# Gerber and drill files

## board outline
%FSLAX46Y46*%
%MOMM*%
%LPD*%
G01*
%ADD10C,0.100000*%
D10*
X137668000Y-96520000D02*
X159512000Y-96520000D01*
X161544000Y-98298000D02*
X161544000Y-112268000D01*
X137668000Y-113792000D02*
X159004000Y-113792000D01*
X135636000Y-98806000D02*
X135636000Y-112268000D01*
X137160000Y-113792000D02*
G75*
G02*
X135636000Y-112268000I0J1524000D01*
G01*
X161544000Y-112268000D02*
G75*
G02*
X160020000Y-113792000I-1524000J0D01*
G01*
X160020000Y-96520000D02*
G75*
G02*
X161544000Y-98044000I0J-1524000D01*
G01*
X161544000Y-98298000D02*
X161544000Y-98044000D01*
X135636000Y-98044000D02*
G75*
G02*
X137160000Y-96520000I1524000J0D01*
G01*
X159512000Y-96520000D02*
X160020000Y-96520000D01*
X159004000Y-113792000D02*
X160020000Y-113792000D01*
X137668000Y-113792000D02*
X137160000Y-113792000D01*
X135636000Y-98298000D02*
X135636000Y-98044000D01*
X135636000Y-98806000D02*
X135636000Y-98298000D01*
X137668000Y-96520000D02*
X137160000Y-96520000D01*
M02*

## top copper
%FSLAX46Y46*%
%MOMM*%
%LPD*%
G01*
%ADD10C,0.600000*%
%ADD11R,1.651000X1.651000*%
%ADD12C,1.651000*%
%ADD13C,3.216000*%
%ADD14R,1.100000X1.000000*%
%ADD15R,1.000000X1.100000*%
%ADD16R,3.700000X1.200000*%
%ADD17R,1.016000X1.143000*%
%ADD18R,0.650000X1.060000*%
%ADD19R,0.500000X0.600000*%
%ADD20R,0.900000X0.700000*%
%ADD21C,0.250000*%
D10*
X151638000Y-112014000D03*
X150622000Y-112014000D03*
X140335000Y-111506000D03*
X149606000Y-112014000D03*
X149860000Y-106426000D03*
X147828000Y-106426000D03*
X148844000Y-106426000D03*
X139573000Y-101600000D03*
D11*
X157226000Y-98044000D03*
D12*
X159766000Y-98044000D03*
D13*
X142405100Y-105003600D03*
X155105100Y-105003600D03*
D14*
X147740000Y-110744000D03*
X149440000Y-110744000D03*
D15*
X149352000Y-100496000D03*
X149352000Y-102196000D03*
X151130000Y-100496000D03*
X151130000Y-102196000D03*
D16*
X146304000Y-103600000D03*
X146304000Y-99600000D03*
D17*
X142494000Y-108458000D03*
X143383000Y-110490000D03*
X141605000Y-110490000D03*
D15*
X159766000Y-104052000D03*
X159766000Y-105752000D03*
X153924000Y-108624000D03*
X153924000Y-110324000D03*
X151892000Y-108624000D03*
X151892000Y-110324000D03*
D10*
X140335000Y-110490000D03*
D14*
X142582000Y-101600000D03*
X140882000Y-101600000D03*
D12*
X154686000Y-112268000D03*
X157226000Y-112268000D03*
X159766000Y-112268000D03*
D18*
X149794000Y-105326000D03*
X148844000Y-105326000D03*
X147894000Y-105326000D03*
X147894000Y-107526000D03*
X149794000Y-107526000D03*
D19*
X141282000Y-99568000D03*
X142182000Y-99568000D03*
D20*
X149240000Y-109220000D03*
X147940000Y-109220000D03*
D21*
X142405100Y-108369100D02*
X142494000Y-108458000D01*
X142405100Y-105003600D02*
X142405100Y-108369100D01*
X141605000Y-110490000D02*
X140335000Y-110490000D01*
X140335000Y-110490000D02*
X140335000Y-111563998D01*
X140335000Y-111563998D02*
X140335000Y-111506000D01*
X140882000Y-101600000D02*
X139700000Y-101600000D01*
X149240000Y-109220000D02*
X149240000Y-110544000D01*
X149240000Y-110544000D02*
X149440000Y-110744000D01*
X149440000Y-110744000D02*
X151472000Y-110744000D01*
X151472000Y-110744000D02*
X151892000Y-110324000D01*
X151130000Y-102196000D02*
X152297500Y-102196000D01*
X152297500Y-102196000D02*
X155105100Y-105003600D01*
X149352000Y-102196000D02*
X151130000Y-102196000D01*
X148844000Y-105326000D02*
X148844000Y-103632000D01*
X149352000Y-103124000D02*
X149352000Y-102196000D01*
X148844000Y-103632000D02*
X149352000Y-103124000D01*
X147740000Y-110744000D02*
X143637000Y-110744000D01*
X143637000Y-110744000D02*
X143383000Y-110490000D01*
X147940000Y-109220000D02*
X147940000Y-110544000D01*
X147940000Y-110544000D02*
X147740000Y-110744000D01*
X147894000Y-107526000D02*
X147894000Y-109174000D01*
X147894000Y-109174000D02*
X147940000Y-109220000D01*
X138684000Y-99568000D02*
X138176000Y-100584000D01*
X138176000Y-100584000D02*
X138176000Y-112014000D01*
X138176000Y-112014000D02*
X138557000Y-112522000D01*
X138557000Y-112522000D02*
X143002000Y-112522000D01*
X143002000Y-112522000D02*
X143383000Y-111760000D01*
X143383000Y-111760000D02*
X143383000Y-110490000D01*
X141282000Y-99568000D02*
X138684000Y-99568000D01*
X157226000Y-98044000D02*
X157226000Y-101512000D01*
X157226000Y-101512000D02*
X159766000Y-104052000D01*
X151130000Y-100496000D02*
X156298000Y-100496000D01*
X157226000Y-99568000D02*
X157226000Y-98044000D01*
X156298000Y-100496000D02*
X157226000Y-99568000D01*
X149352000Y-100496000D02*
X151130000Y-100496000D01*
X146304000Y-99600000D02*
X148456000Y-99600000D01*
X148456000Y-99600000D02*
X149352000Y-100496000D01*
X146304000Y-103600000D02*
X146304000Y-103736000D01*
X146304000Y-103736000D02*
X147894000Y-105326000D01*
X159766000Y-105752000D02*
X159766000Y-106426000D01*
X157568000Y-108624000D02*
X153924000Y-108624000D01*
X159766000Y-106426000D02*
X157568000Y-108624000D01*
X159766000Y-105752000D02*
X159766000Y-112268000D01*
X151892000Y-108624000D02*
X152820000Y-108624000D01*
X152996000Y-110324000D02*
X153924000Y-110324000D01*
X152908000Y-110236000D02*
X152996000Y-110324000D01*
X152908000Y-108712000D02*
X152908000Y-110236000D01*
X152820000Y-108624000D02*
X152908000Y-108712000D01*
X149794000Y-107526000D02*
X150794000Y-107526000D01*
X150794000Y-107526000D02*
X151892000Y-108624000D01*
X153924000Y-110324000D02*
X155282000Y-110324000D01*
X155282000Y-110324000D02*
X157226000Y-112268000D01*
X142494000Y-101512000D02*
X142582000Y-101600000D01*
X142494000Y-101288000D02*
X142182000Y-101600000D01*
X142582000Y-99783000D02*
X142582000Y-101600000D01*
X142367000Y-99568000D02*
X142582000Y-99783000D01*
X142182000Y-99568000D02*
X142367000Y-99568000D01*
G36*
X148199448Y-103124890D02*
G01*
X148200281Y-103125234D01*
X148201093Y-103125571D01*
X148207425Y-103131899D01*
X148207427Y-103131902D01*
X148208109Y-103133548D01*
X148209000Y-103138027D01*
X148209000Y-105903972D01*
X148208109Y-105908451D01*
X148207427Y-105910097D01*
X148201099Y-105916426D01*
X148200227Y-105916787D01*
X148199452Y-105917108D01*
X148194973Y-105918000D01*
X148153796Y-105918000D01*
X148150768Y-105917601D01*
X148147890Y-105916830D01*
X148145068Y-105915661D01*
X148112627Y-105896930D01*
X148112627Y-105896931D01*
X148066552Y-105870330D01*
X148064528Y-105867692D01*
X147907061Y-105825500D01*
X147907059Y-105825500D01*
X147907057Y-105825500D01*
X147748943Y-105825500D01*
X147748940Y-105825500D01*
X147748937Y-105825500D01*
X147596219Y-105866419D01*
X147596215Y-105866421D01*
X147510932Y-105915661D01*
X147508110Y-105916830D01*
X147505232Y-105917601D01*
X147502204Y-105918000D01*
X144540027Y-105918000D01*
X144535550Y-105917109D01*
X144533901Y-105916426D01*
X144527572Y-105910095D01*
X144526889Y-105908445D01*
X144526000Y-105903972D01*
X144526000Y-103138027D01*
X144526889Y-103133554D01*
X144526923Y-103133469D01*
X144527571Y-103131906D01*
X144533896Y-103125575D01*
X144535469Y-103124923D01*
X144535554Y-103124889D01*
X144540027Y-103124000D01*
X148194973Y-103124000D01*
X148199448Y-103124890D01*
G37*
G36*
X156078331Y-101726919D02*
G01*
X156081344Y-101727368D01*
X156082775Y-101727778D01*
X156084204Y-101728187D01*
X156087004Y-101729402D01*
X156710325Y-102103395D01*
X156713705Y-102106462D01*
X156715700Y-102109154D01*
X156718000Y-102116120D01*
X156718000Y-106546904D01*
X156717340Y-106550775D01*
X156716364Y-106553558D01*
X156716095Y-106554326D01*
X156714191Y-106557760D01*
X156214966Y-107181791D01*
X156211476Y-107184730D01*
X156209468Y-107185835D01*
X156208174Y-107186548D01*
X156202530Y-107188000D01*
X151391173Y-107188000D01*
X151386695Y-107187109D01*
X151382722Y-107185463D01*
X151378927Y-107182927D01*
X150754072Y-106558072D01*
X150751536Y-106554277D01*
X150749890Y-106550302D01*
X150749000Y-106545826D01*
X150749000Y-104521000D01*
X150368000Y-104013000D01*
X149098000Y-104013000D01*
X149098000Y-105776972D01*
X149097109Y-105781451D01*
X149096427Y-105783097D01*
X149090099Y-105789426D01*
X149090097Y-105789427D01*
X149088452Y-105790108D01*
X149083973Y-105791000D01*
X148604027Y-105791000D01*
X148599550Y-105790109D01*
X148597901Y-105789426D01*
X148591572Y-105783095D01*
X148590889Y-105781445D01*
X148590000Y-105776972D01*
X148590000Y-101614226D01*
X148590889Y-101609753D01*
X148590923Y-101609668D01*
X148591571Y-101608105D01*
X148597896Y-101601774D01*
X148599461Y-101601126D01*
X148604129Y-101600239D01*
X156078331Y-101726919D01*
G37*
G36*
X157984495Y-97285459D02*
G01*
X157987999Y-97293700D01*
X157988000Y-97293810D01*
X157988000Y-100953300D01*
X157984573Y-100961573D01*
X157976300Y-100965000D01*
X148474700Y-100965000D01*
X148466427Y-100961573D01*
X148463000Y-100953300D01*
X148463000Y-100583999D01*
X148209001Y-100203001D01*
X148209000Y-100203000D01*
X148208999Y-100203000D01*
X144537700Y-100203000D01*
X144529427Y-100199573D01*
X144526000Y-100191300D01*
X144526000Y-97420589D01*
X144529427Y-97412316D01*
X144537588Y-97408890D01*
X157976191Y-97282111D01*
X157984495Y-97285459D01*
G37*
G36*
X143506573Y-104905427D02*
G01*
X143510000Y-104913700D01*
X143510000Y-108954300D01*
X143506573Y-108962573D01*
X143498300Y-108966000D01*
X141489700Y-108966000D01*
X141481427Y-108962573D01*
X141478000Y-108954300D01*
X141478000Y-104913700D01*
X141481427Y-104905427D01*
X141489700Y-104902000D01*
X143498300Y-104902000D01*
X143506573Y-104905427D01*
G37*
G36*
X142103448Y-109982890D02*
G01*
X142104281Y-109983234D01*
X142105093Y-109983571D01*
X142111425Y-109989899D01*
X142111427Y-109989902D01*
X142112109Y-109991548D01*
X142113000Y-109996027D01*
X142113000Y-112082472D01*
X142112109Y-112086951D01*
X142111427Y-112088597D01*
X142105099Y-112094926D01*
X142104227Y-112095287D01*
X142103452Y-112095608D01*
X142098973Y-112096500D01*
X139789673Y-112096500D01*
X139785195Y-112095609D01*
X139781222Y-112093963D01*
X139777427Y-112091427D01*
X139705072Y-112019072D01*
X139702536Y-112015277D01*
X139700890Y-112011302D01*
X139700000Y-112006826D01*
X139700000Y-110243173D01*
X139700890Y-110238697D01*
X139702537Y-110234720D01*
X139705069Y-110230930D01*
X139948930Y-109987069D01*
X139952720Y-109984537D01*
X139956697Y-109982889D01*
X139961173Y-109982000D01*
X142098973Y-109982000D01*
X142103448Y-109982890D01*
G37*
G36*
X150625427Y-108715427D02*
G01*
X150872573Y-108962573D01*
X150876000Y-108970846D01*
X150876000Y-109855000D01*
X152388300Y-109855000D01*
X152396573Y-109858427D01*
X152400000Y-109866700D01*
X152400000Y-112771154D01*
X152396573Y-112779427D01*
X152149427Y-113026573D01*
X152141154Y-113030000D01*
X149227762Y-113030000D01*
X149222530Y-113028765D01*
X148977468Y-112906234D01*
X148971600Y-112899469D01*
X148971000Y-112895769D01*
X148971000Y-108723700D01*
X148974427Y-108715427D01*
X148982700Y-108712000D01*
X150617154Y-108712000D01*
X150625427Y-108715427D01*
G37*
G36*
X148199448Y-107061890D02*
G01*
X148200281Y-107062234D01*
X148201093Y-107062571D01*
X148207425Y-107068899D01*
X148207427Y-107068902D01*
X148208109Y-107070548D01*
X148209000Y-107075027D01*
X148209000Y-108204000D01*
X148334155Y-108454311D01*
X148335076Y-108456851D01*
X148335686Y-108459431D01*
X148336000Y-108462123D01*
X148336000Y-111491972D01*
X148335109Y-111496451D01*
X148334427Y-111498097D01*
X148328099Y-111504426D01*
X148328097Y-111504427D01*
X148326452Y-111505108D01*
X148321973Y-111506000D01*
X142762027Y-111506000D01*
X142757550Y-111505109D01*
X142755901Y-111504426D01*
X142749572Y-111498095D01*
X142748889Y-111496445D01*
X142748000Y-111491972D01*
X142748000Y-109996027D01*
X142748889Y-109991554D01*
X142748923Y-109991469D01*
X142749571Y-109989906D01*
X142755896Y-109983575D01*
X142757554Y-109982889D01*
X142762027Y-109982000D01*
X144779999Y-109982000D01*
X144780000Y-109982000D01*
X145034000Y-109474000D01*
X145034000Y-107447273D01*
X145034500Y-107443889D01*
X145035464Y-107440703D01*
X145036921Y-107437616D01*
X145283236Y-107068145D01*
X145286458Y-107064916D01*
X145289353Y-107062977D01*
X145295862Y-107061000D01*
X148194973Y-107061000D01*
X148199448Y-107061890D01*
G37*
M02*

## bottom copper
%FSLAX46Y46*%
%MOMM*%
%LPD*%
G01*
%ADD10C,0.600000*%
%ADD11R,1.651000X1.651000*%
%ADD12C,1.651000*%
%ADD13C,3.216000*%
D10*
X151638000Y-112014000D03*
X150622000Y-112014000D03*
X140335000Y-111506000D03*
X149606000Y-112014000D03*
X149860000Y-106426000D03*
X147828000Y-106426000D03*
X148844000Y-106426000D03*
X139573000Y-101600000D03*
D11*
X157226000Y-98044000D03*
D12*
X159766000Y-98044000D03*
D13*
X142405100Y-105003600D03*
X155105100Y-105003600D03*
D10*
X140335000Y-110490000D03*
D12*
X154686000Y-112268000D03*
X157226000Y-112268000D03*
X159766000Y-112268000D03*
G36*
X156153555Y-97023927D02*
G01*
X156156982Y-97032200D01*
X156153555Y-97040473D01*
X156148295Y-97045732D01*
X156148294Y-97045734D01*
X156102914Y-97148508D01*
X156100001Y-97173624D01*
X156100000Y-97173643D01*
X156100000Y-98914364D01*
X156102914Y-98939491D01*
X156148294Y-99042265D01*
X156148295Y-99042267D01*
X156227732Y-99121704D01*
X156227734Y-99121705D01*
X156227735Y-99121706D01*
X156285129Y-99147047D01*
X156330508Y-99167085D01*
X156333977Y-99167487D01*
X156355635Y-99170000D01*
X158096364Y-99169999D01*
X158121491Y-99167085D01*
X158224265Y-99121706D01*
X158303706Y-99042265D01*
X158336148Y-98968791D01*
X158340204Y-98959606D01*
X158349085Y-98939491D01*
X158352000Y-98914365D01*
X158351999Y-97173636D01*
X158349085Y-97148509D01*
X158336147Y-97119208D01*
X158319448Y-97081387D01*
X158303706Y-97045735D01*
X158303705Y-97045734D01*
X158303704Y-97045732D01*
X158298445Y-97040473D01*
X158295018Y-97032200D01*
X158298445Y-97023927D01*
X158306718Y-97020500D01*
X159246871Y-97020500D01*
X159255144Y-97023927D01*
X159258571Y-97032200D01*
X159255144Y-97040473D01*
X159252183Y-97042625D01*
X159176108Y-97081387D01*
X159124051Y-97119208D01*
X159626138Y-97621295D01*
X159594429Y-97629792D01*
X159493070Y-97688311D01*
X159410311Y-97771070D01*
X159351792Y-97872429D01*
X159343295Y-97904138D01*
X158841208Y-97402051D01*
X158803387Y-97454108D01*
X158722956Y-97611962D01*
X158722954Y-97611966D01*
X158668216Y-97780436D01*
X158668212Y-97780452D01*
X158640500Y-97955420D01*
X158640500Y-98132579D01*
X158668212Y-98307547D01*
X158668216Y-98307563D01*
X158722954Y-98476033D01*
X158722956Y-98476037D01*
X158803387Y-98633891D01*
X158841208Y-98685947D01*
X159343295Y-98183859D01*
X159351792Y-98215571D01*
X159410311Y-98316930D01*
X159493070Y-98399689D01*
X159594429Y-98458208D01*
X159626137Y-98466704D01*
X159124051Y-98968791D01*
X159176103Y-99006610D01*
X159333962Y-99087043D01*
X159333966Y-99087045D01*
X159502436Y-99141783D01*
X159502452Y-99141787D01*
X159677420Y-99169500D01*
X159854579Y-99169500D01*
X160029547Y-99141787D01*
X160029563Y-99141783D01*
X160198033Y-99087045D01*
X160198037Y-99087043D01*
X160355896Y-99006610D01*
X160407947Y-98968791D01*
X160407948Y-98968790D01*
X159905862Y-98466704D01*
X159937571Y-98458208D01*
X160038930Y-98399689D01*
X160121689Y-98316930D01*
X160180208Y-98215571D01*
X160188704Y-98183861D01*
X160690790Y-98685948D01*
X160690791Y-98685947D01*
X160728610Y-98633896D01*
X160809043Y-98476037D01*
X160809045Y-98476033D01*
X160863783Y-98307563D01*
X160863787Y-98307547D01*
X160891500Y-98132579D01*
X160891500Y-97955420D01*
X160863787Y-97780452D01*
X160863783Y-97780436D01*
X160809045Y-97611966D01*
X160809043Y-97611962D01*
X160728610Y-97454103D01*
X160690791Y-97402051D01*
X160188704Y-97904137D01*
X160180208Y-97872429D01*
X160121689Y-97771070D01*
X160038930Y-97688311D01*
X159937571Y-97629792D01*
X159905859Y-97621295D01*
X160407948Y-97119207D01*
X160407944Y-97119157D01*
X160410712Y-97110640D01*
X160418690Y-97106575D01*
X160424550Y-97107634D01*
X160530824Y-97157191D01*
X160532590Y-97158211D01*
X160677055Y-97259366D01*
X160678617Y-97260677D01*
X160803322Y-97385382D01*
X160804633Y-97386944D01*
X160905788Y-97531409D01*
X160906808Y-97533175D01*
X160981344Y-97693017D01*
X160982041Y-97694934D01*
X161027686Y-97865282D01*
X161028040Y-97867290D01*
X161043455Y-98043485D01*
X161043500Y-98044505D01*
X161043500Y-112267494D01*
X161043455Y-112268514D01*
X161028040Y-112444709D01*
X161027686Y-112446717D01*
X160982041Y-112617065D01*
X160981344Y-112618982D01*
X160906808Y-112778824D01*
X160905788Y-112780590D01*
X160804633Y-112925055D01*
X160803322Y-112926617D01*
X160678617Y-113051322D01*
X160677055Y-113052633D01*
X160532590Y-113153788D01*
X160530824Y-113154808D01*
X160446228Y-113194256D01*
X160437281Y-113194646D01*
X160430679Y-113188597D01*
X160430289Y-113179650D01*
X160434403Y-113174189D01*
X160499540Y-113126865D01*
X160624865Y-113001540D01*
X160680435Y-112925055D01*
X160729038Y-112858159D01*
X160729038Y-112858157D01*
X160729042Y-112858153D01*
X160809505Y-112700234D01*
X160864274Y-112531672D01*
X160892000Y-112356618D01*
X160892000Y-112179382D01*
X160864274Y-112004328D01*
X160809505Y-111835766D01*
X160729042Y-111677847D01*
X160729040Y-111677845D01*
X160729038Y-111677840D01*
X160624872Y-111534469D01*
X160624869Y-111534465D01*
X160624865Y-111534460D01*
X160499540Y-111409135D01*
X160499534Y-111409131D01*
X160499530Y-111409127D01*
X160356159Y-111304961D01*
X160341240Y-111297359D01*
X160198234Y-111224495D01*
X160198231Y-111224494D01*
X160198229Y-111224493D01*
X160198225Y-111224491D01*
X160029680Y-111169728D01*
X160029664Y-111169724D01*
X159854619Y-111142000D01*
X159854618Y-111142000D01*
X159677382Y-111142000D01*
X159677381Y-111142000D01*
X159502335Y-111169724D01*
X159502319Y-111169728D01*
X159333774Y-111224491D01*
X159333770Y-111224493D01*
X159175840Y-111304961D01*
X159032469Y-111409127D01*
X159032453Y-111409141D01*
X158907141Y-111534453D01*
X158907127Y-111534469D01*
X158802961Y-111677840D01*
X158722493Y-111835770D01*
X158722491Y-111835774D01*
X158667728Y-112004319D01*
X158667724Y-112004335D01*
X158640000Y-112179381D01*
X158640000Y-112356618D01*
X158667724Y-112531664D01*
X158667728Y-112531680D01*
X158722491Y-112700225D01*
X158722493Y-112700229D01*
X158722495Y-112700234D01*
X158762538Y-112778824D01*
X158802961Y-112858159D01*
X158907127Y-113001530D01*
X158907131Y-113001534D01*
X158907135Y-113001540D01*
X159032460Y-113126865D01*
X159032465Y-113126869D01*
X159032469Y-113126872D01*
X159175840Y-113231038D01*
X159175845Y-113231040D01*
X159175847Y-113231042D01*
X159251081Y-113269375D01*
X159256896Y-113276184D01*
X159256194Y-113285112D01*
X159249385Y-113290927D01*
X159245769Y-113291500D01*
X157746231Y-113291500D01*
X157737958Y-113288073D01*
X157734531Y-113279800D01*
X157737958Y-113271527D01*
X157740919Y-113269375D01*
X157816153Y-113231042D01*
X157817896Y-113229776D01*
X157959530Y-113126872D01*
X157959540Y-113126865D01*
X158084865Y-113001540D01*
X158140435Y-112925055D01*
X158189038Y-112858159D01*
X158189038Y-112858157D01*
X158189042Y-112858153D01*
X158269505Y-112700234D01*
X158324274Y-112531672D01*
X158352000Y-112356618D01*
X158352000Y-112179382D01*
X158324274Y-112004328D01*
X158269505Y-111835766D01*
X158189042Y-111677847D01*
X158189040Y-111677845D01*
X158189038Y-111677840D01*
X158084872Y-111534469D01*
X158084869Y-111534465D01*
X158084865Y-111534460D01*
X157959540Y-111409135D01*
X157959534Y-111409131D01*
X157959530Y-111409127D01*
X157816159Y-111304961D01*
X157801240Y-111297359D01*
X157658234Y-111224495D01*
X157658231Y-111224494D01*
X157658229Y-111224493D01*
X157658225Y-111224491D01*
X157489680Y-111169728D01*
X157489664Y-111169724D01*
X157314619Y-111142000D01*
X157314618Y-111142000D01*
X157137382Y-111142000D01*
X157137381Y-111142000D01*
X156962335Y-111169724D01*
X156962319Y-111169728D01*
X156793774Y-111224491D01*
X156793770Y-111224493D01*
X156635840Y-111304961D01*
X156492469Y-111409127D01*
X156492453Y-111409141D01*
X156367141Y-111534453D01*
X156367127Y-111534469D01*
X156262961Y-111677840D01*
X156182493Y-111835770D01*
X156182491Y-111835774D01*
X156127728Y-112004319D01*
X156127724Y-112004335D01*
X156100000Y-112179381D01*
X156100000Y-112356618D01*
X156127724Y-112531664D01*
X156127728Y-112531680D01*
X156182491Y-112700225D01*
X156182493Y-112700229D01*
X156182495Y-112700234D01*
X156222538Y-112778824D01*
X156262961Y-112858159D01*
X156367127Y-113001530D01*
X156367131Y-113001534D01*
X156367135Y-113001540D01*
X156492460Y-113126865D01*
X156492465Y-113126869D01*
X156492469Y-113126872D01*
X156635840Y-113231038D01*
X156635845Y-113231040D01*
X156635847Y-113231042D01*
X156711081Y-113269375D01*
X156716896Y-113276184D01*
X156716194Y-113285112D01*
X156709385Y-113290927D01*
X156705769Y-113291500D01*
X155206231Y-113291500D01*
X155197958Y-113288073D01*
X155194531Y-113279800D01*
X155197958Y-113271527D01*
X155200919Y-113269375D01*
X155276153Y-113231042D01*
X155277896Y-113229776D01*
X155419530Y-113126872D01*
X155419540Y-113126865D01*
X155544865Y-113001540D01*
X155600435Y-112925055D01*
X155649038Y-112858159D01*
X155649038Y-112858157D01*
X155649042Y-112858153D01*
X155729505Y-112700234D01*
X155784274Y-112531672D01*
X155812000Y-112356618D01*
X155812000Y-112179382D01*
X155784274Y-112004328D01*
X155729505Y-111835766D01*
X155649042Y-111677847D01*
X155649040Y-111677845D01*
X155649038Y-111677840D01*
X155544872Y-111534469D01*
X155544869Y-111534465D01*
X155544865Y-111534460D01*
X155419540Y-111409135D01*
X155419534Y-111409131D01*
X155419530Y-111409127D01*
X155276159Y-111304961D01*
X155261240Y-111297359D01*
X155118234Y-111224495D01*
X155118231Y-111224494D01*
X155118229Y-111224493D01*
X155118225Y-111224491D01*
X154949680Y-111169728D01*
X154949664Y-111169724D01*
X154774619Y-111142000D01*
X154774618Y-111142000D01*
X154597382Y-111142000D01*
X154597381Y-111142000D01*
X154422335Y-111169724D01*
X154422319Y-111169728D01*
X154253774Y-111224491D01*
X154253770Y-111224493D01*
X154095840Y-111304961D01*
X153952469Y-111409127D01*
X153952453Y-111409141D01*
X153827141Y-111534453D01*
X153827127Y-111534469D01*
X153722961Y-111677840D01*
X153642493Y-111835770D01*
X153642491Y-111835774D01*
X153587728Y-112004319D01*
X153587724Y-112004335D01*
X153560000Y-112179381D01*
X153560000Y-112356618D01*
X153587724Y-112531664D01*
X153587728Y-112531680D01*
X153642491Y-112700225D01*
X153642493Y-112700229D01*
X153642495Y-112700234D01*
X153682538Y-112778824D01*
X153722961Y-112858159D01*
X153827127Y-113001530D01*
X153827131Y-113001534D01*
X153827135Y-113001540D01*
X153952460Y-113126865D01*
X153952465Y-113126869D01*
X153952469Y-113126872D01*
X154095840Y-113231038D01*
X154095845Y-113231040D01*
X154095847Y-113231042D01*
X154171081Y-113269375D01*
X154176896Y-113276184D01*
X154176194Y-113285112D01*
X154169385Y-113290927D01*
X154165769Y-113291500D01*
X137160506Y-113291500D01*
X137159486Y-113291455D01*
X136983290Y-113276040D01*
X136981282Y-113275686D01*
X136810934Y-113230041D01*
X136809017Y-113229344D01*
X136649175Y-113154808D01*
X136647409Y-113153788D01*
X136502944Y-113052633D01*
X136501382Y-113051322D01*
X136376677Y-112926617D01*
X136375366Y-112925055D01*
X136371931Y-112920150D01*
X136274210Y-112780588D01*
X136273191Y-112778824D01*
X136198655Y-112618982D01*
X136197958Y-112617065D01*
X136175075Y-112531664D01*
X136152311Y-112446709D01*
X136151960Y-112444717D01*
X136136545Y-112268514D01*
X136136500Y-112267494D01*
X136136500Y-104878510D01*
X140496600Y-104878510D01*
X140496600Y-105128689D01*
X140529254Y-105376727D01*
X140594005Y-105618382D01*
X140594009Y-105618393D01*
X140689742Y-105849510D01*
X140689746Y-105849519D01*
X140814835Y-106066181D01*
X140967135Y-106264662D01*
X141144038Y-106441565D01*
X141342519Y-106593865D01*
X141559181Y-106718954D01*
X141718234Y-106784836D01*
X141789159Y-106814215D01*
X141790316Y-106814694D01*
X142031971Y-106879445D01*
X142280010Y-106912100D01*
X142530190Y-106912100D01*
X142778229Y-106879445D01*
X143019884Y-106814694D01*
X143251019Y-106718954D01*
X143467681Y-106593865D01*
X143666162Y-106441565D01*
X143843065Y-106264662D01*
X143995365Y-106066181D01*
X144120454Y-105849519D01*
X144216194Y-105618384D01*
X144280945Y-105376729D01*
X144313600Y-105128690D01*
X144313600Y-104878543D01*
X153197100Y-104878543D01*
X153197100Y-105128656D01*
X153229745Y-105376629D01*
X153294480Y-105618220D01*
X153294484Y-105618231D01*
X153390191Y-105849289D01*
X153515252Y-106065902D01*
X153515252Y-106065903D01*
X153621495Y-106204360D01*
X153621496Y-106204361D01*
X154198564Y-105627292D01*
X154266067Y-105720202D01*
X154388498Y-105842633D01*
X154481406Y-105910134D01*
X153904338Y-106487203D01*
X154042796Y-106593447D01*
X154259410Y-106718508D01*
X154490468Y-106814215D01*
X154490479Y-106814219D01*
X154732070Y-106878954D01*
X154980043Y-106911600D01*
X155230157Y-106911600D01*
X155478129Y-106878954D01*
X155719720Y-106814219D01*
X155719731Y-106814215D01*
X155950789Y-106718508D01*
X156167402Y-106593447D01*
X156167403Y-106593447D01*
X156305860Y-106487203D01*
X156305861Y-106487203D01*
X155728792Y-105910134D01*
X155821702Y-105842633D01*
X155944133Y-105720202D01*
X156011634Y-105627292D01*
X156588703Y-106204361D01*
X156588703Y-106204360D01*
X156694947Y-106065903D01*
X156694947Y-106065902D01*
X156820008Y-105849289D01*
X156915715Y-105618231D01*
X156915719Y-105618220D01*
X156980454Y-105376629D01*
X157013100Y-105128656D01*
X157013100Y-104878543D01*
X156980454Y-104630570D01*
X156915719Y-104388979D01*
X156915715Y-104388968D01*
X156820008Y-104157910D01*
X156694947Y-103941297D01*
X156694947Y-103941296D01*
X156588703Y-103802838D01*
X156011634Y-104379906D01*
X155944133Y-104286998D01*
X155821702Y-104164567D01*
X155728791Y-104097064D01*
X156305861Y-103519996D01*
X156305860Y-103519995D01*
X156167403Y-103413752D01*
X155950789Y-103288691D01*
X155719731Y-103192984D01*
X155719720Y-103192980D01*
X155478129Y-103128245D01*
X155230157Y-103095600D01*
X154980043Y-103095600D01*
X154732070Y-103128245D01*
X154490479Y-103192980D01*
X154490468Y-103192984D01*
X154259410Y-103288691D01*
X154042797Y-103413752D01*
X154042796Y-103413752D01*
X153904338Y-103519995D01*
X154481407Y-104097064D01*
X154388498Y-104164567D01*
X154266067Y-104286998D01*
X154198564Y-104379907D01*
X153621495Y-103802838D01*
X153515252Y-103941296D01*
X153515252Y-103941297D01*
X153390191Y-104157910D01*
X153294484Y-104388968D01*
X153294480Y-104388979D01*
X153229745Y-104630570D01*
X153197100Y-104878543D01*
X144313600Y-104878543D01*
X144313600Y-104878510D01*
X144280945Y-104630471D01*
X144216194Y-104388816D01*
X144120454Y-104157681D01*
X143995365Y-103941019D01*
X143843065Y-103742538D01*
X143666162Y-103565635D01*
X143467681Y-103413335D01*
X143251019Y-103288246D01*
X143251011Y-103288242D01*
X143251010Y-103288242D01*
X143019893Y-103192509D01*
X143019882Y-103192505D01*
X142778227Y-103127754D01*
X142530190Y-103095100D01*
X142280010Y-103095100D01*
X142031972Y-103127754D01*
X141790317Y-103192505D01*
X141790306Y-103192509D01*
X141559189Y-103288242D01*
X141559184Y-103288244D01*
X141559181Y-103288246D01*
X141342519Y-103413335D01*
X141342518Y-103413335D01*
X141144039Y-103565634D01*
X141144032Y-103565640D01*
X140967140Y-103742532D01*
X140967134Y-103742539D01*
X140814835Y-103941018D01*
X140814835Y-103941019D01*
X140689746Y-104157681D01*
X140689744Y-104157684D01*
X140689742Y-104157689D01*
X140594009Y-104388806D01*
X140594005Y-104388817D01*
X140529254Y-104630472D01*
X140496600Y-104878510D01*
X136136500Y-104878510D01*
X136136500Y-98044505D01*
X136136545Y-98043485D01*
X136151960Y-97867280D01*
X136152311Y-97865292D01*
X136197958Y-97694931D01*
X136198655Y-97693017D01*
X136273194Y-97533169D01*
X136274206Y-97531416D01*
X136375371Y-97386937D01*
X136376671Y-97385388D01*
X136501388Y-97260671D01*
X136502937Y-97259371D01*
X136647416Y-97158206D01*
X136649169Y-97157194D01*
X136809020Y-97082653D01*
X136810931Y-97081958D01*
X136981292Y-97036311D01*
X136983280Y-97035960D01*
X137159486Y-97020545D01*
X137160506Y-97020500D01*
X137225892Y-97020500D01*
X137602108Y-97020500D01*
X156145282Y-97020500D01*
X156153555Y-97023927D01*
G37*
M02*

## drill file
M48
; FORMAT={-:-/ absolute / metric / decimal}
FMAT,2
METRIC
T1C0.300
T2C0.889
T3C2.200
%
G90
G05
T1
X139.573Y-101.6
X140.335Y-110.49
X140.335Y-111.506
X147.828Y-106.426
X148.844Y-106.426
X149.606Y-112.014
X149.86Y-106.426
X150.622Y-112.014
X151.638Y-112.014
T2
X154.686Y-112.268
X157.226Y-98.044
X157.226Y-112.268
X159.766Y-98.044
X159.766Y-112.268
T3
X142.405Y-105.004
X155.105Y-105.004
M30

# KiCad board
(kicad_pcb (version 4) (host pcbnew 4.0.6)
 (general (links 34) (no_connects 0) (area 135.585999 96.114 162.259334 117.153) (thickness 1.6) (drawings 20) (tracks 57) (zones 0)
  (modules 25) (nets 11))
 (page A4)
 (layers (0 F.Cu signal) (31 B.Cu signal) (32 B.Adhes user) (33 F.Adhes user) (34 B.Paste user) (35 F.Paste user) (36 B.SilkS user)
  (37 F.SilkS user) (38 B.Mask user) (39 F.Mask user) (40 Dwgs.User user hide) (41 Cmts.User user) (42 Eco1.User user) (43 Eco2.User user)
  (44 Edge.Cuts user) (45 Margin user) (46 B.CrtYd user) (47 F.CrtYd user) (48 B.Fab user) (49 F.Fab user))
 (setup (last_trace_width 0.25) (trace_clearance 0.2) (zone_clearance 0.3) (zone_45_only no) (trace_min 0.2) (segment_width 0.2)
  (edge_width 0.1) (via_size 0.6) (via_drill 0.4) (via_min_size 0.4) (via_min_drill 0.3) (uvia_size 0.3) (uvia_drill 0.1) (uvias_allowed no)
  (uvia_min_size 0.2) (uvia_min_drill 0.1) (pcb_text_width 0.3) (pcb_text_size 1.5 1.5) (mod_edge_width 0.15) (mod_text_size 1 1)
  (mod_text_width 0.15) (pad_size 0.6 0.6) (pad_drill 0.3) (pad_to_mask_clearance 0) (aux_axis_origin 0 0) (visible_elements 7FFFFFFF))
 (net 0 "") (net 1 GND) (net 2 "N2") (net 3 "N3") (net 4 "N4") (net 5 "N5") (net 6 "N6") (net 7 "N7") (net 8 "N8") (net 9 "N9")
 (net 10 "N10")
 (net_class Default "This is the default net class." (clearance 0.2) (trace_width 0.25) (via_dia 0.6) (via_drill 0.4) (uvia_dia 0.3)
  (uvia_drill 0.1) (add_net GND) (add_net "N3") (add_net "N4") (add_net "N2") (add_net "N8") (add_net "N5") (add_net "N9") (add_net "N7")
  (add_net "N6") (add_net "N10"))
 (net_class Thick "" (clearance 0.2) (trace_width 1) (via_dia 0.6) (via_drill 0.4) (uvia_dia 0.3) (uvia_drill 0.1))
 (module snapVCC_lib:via (layer F.Cu) (at 151.638 112.014)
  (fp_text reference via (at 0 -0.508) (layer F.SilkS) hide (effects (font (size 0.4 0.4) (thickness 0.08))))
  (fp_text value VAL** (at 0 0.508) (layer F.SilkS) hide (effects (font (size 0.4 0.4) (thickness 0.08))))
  (pad 1 thru_hole circle (at 0 0) (size 0.6 0.6) (drill 0.3) (layers *.Cu) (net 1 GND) (zone_connect 2)))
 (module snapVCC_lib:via (layer F.Cu) (at 150.622 112.014)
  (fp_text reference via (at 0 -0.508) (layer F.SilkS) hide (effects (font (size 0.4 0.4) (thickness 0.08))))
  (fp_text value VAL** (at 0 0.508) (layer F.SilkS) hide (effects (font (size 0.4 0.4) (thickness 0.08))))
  (pad 1 thru_hole circle (at 0 0) (size 0.6 0.6) (drill 0.3) (layers *.Cu) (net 1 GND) (zone_connect 2)))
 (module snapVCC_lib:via (layer F.Cu) (at 140.335 111.506)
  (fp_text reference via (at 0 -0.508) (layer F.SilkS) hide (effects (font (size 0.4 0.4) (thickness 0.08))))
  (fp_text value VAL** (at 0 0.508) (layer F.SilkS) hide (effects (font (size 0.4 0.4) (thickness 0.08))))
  (pad 1 thru_hole circle (at 0 0) (size 0.6 0.6) (drill 0.3) (layers *.Cu) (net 1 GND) (zone_connect 2)))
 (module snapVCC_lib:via (layer F.Cu) (at 149.606 112.014)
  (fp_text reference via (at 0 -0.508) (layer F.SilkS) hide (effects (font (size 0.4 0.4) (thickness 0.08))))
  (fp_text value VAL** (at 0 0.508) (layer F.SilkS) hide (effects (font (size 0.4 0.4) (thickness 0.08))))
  (pad 1 thru_hole circle (at 0 0) (size 0.6 0.6) (drill 0.3) (layers *.Cu) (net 1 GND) (zone_connect 2)))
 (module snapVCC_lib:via (layer F.Cu) (at 149.86 106.426)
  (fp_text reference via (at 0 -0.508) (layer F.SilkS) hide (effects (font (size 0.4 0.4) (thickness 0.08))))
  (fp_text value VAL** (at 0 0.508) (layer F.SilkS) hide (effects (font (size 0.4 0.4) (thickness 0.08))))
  (pad 1 thru_hole circle (at 0 0) (size 0.6 0.6) (drill 0.3) (layers *.Cu) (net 1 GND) (zone_connect 2)))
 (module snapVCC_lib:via (layer F.Cu) (at 147.828 106.426)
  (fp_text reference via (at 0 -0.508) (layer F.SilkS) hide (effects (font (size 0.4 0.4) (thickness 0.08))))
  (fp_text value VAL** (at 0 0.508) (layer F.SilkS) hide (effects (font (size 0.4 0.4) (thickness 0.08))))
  (pad 1 thru_hole circle (at 0 0) (size 0.6 0.6) (drill 0.3) (layers *.Cu) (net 1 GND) (zone_connect 2)))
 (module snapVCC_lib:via (layer F.Cu) (at 148.844 106.426)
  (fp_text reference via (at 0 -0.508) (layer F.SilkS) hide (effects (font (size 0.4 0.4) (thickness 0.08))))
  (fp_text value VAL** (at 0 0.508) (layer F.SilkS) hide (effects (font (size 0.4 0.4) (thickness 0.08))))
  (pad 1 thru_hole circle (at 0 0) (size 0.6 0.6) (drill 0.3) (layers *.Cu) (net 1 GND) (zone_connect 2)))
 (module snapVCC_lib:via (layer F.Cu) (at 139.573 101.6)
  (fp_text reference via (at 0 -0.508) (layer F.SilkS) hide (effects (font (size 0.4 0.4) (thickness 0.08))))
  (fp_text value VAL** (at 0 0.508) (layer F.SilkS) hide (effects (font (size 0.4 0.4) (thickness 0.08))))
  (pad 1 thru_hole circle (at 0 0) (size 0.6 0.6) (drill 0.3) (layers *.Cu) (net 1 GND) (zone_connect 2)))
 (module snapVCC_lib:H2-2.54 (layer F.Cu) (at 158.496 98.044 90)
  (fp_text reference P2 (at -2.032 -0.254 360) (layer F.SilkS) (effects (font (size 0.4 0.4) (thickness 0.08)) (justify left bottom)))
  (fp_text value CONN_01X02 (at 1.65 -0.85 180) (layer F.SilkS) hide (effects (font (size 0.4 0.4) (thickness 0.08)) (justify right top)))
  (pad 1 thru_hole rect (at 0 -1.27 90) (size 1.651 1.651) (drill 0.889) (layers *.Cu *.Mask) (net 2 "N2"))
  (pad 2 thru_hole circle (at 0 1.27 90) (size 1.651 1.651) (drill 0.889) (layers *.Cu *.Mask) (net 1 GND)))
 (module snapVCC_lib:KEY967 (layer B.Cu) (at 148.7551 105.0036)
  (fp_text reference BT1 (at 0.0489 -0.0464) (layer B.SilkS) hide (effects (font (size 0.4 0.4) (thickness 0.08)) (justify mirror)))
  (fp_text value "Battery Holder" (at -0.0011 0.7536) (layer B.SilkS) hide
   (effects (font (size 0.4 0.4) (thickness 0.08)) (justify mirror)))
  (pad 1 thru_hole circle (at -6.35 0) (size 3.216 3.216) (drill 2.2) (layers *.Cu *.Mask) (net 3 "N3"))
  (pad 2 thru_hole circle (at 6.35 0) (size 3.216 3.216) (drill 2.2) (layers *.Cu *.Mask) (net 1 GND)))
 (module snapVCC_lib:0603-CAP (layer F.Cu) (at 148.59 110.744)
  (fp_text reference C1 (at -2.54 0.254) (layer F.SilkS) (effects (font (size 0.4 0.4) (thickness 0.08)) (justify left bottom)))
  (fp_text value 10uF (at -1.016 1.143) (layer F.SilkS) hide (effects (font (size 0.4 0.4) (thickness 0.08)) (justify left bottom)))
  (pad 1 smd rect (at -0.85 0) (size 1.1 1) (layers F.Cu F.Paste F.Mask) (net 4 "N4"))
  (pad 2 smd rect (at 0.85 0) (size 1.1 1) (layers F.Cu F.Paste F.Mask) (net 1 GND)))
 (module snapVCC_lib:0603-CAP (layer F.Cu) (at 149.352 101.346 270)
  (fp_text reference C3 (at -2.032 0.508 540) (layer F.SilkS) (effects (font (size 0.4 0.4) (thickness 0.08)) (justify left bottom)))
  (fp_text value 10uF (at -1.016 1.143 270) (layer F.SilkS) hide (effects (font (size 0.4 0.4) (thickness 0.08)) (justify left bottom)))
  (pad 1 smd rect (at -0.85 0 270) (size 1.1 1) (layers F.Cu F.Paste F.Mask) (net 2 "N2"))
  (pad 2 smd rect (at 0.85 0 270) (size 1.1 1) (layers F.Cu F.Paste F.Mask) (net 1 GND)))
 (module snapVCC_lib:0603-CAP (layer F.Cu) (at 151.13 101.346 270)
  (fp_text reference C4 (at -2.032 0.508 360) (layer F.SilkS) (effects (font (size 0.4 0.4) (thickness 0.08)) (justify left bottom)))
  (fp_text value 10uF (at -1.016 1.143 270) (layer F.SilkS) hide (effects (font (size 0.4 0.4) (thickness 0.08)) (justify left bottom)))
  (pad 1 smd rect (at -0.85 0 270) (size 1.1 1) (layers F.Cu F.Paste F.Mask) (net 2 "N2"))
  (pad 2 smd rect (at 0.85 0 270) (size 1.1 1) (layers F.Cu F.Paste F.Mask) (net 1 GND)))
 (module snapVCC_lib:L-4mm (layer F.Cu) (at 146.304 101.6 90)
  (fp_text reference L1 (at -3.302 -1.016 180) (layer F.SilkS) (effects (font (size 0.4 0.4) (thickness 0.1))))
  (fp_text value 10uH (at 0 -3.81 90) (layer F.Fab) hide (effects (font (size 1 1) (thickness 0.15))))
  (pad 1 smd rect (at -2 0 90) (size 1.2 3.7) (layers F.Cu F.Paste F.Mask) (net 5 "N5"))
  (pad 2 smd rect (at 2 0 90) (size 1.2 3.7) (layers F.Cu F.Paste F.Mask) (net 2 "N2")))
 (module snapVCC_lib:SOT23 (layer F.Cu) (at 142.494 109.474)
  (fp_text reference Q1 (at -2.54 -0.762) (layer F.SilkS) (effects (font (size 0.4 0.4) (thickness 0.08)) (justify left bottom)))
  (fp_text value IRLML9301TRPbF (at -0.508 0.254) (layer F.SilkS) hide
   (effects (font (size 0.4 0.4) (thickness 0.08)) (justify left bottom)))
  (pad 3 smd rect (at 0 -1.016) (size 1.016 1.143) (layers F.Cu F.Paste F.Mask) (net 3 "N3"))
  (pad 2 smd rect (at 0.889 1.016) (size 1.016 1.143) (layers F.Cu F.Paste F.Mask) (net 4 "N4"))
  (pad 1 smd rect (at -0.889 1.016 180) (size 1.016 1.143) (layers F.Cu F.Paste F.Mask) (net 1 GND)))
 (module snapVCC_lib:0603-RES (layer F.Cu) (at 159.766 104.902 270)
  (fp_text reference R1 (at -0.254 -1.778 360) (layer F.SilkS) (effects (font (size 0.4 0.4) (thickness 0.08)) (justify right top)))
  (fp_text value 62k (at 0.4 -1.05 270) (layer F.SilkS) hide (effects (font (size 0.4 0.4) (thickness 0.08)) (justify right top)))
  (pad 1 smd rect (at -0.85 0 270) (size 1.1 1) (layers F.Cu F.Paste F.Mask) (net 2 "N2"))
  (pad 2 smd rect (at 0.85 0 270) (size 1.1 1) (layers F.Cu F.Paste F.Mask) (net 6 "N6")))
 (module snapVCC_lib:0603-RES (layer F.Cu) (at 153.924 109.474 270)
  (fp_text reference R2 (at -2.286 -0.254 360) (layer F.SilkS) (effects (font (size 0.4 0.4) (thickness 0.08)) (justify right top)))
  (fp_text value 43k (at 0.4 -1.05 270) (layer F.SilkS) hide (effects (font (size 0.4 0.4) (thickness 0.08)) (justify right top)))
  (pad 1 smd rect (at -0.85 0 270) (size 1.1 1) (layers F.Cu F.Paste F.Mask) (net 6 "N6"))
  (pad 2 smd rect (at 0.85 0 270) (size 1.1 1) (layers F.Cu F.Paste F.Mask) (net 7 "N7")))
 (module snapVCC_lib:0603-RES (layer F.Cu) (at 151.892 109.474 270)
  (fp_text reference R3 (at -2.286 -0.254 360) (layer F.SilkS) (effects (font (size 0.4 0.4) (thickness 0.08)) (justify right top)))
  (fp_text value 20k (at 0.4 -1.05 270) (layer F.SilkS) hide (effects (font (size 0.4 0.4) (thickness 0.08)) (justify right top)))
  (pad 1 smd rect (at -0.85 0 270) (size 1.1 1) (layers F.Cu F.Paste F.Mask) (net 7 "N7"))
  (pad 2 smd rect (at 0.85 0 270) (size 1.1 1) (layers F.Cu F.Paste F.Mask) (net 1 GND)))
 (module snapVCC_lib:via (layer F.Cu) (at 140.335 110.49)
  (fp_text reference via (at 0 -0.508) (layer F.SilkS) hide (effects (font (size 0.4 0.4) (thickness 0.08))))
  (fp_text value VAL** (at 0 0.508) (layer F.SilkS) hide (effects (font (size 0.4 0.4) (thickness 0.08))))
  (pad 1 thru_hole circle (at 0 0) (size 0.6 0.6) (drill 0.3) (layers *.Cu) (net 1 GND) (zone_connect 2)))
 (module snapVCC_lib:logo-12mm (layer F.Cu) (at 138.049 105.156 90)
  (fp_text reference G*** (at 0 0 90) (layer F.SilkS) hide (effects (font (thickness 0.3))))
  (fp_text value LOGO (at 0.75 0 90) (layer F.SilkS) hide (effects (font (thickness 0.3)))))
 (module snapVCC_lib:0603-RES (layer F.Cu) (at 141.732 101.6 180)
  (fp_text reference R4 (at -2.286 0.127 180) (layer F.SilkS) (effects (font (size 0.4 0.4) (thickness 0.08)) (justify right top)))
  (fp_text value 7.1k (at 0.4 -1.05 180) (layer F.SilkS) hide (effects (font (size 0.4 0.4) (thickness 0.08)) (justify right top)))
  (pad 1 smd rect (at -0.85 0 180) (size 1.1 1) (layers F.Cu F.Paste F.Mask) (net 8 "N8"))
  (pad 2 smd rect (at 0.85 0 180) (size 1.1 1) (layers F.Cu F.Paste F.Mask) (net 1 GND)))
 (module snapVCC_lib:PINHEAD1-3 (layer F.Cu) (at 157.226 112.268)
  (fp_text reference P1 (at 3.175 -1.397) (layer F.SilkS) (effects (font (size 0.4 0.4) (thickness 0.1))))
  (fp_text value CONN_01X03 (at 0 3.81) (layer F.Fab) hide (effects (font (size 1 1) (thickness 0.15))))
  (pad 1 thru_hole circle (at -2.54 0) (size 1.651 1.651) (drill 0.889) (layers *.Cu *.Mask) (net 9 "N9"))
  (pad 2 thru_hole circle (at 0 0) (size 1.651 1.651) (drill 0.889) (layers *.Cu *.Mask) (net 7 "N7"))
  (pad 3 thru_hole circle (at 2.54 0) (size 1.651 1.651) (drill 0.889) (layers *.Cu *.Mask) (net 6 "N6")))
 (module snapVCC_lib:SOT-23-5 (layer F.Cu) (at 148.844 106.426 270)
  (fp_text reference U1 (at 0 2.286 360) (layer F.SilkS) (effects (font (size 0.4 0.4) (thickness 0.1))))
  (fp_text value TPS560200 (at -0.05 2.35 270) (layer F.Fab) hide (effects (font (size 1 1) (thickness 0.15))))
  (pad 1 smd rect (at -1.1 -0.95 270) (size 1.06 0.65) (layers F.Cu F.Paste F.Mask) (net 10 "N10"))
  (pad 2 smd rect (at -1.1 0 270) (size 1.06 0.65) (layers F.Cu F.Paste F.Mask) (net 1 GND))
  (pad 3 smd rect (at -1.1 0.95 270) (size 1.06 0.65) (layers F.Cu F.Paste F.Mask) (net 5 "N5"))
  (pad 4 smd rect (at 1.1 0.95 270) (size 1.06 0.65) (layers F.Cu F.Paste F.Mask) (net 4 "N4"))
  (pad 5 smd rect (at 1.1 -0.95 270) (size 1.06 0.65) (layers F.Cu F.Paste F.Mask) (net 7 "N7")))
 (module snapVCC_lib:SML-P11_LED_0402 (layer F.Cu) (at 141.732 99.568 180)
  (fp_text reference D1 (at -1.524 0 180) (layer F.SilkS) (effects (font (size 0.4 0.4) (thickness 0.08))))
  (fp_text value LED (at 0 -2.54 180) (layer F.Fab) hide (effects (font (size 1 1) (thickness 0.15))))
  (pad 2 smd rect (at 0.45 0 180) (size 0.5 0.6) (layers F.Cu F.Paste F.Mask) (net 4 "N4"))
  (pad 1 smd rect (at -0.45 0 180) (size 0.5 0.6) (layers F.Cu F.Paste F.Mask) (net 8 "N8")))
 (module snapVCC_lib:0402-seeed (layer F.Cu) (at 148.59 109.22)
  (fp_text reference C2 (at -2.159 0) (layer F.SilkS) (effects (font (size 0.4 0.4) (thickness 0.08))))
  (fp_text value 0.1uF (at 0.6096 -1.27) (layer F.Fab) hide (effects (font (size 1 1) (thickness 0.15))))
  (pad 2 smd rect (at 0.65 0) (size 0.9 0.7) (layers F.Cu F.Paste F.Mask) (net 1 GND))
  (pad 1 smd rect (at -0.65 0) (size 0.9 0.7) (layers F.Cu F.Paste F.Mask) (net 4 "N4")))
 (gr_line (start 137.668 96.52) (end 159.512 96.52) (angle 90) (layer Edge.Cuts) (width 0.1))
 (gr_line (start 161.544 98.298) (end 161.544 112.268) (angle 90) (layer Edge.Cuts) (width 0.1))
 (gr_line (start 137.668 113.792) (end 159.004 113.792) (angle 90) (layer Edge.Cuts) (width 0.1))
 (gr_line (start 135.636 98.806) (end 135.636 112.268) (angle 90) (layer Edge.Cuts) (width 0.1))
 (gr_arc (start 137.16 112.268) (end 137.16 113.792) (angle 90) (layer Edge.Cuts) (width 0.1))
 (gr_arc (start 160.02 112.268) (end 161.544 112.268) (angle 90) (layer Edge.Cuts) (width 0.1))
 (gr_arc (start 160.02 98.044) (end 160.02 96.52) (angle 90) (layer Edge.Cuts) (width 0.1))
 (gr_line (start 161.544 98.298) (end 161.544 98.044) (angle 90) (layer Edge.Cuts) (width 0.1))
 (gr_arc (start 137.16 98.044) (end 135.636 98.044) (angle 90) (layer Edge.Cuts) (width 0.1))
 (gr_line (start 159.512 96.52) (end 160.02 96.52) (angle 90) (layer Edge.Cuts) (width 0.1))
 (gr_line (start 159.004 113.792) (end 160.02 113.792) (angle 90) (layer Edge.Cuts) (width 0.1))
 (gr_line (start 137.668 113.792) (end 137.16 113.792) (angle 90) (layer Edge.Cuts) (width 0.1))
 (gr_line (start 135.636 98.298) (end 135.636 98.044) (angle 90) (layer Edge.Cuts) (width 0.1))
 (gr_line (start 135.636 98.806) (end 135.636 98.298) (angle 90) (layer Edge.Cuts) (width 0.1))
 (gr_line (start 137.668 96.52) (end 137.16 96.52) (angle 90) (layer Edge.Cuts) (width 0.1))
 (segment (start 142.4051 108.3691) (end 142.494 108.458) (width 0.25) (layer F.Cu) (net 3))
 (segment (start 142.4051 105.0036) (end 142.4051 108.3691) (width 0.25) (layer F.Cu) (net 3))
 (segment (start 141.605 110.49) (end 140.335 110.49) (width 0.25) (layer F.Cu) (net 1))
 (segment (start 140.335 110.49) (end 140.335 111.563998) (width 0.25) (layer F.Cu) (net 1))
 (segment (start 140.335 111.563998) (end 140.335 111.506) (width 0.25) (layer F.Cu) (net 1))
 (segment (start 140.882 101.6) (end 139.7 101.6) (width 0.25) (layer F.Cu) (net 1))
 (segment (start 149.24 109.22) (end 149.24 110.544) (width 0.25) (layer F.Cu) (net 1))
 (segment (start 149.24 110.544) (end 149.44 110.744) (width 0.25) (layer F.Cu) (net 1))
 (segment (start 149.44 110.744) (end 151.472 110.744) (width 0.25) (layer F.Cu) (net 1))
 (segment (start 151.472 110.744) (end 151.892 110.324) (width 0.25) (layer F.Cu) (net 1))
 (segment (start 151.13 102.196) (end 152.2975 102.196) (width 0.25) (layer F.Cu) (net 1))
 (segment (start 152.2975 102.196) (end 155.1051 105.0036) (width 0.25) (layer F.Cu) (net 1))
 (segment (start 149.352 102.196) (end 151.13 102.196) (width 0.25) (layer F.Cu) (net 1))
 (segment (start 148.844 105.326) (end 148.844 103.632) (width 0.25) (layer F.Cu) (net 1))
 (segment (start 149.352 103.124) (end 149.352 102.196) (width 0.25) (layer F.Cu) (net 1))
 (segment (start 148.844 103.632) (end 149.352 103.124) (width 0.25) (layer F.Cu) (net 1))
 (segment (start 147.74 110.744) (end 143.637 110.744) (width 0.25) (layer F.Cu) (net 4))
 (segment (start 143.637 110.744) (end 143.383 110.49) (width 0.25) (layer F.Cu) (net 4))
 (segment (start 147.94 109.22) (end 147.94 110.544) (width 0.25) (layer F.Cu) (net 4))
 (segment (start 147.94 110.544) (end 147.74 110.744) (width 0.25) (layer F.Cu) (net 4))
 (segment (start 147.894 107.526) (end 147.894 109.174) (width 0.25) (layer F.Cu) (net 4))
 (segment (start 147.894 109.174) (end 147.94 109.22) (width 0.25) (layer F.Cu) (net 4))
 (segment (start 138.684 99.568) (end 138.176 100.584) (width 0.25) (layer F.Cu) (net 4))
 (segment (start 138.176 100.584) (end 138.176 112.014) (width 0.25) (layer F.Cu) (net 4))
 (segment (start 138.176 112.014) (end 138.557 112.522) (width 0.25) (layer F.Cu) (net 4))
 (segment (start 138.557 112.522) (end 143.002 112.522) (width 0.25) (layer F.Cu) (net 4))
 (segment (start 143.002 112.522) (end 143.383 111.76) (width 0.25) (layer F.Cu) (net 4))
 (segment (start 143.383 111.76) (end 143.383 110.49) (width 0.25) (layer F.Cu) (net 4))
 (segment (start 141.282 99.568) (end 138.684 99.568) (width 0.25) (layer F.Cu) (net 4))
 (segment (start 157.226 98.044) (end 157.226 101.512) (width 0.25) (layer F.Cu) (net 2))
 (segment (start 157.226 101.512) (end 159.766 104.052) (width 0.25) (layer F.Cu) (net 2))
 (segment (start 151.13 100.496) (end 156.298 100.496) (width 0.25) (layer F.Cu) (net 2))
 (segment (start 157.226 99.568) (end 157.226 98.044) (width 0.25) (layer F.Cu) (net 2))
 (segment (start 156.298 100.496) (end 157.226 99.568) (width 0.25) (layer F.Cu) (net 2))
 (segment (start 149.352 100.496) (end 151.13 100.496) (width 0.25) (layer F.Cu) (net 2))
 (segment (start 146.304 99.6) (end 148.456 99.6) (width 0.25) (layer F.Cu) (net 2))
 (segment (start 148.456 99.6) (end 149.352 100.496) (width 0.25) (layer F.Cu) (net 2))
 (segment (start 146.304 103.6) (end 146.304 103.736) (width 0.25) (layer F.Cu) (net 5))
 (segment (start 146.304 103.736) (end 147.894 105.326) (width 0.25) (layer F.Cu) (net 5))
 (segment (start 159.766 105.752) (end 159.766 106.426) (width 0.25) (layer F.Cu) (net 6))
 (segment (start 157.568 108.624) (end 153.924 108.624) (width 0.25) (layer F.Cu) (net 6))
 (segment (start 159.766 106.426) (end 157.568 108.624) (width 0.25) (layer F.Cu) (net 6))
 (segment (start 159.766 105.752) (end 159.766 112.268) (width 0.25) (layer F.Cu) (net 6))
 (segment (start 151.892 108.624) (end 152.82 108.624) (width 0.25) (layer F.Cu) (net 7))
 (segment (start 152.996 110.324) (end 153.924 110.324) (width 0.25) (layer F.Cu) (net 7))
 (segment (start 152.908 110.236) (end 152.996 110.324) (width 0.25) (layer F.Cu) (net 7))
 (segment (start 152.908 108.712) (end 152.908 110.236) (width 0.25) (layer F.Cu) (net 7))
 (segment (start 152.82 108.624) (end 152.908 108.712) (width 0.25) (layer F.Cu) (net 7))
 (segment (start 149.794 107.526) (end 150.794 107.526) (width 0.25) (layer F.Cu) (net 7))
 (segment (start 150.794 107.526) (end 151.892 108.624) (width 0.25) (layer F.Cu) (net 7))
 (segment (start 153.924 110.324) (end 155.282 110.324) (width 0.25) (layer F.Cu) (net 7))
 (segment (start 155.282 110.324) (end 157.226 112.268) (width 0.25) (layer F.Cu) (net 7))
 (segment (start 142.494 101.512) (end 142.582 101.6) (width 0.25) (layer F.Cu) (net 8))
 (segment (start 142.494 101.288) (end 142.182 101.6) (width 0.25) (layer F.Cu) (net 8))
 (segment (start 142.582 99.783) (end 142.582 101.6) (width 0.25) (layer F.Cu) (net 8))
 (segment (start 142.367 99.568) (end 142.582 99.783) (width 0.25) (layer F.Cu) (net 8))
 (segment (start 142.182 99.568) (end 142.367 99.568) (width 0.25) (layer F.Cu) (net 8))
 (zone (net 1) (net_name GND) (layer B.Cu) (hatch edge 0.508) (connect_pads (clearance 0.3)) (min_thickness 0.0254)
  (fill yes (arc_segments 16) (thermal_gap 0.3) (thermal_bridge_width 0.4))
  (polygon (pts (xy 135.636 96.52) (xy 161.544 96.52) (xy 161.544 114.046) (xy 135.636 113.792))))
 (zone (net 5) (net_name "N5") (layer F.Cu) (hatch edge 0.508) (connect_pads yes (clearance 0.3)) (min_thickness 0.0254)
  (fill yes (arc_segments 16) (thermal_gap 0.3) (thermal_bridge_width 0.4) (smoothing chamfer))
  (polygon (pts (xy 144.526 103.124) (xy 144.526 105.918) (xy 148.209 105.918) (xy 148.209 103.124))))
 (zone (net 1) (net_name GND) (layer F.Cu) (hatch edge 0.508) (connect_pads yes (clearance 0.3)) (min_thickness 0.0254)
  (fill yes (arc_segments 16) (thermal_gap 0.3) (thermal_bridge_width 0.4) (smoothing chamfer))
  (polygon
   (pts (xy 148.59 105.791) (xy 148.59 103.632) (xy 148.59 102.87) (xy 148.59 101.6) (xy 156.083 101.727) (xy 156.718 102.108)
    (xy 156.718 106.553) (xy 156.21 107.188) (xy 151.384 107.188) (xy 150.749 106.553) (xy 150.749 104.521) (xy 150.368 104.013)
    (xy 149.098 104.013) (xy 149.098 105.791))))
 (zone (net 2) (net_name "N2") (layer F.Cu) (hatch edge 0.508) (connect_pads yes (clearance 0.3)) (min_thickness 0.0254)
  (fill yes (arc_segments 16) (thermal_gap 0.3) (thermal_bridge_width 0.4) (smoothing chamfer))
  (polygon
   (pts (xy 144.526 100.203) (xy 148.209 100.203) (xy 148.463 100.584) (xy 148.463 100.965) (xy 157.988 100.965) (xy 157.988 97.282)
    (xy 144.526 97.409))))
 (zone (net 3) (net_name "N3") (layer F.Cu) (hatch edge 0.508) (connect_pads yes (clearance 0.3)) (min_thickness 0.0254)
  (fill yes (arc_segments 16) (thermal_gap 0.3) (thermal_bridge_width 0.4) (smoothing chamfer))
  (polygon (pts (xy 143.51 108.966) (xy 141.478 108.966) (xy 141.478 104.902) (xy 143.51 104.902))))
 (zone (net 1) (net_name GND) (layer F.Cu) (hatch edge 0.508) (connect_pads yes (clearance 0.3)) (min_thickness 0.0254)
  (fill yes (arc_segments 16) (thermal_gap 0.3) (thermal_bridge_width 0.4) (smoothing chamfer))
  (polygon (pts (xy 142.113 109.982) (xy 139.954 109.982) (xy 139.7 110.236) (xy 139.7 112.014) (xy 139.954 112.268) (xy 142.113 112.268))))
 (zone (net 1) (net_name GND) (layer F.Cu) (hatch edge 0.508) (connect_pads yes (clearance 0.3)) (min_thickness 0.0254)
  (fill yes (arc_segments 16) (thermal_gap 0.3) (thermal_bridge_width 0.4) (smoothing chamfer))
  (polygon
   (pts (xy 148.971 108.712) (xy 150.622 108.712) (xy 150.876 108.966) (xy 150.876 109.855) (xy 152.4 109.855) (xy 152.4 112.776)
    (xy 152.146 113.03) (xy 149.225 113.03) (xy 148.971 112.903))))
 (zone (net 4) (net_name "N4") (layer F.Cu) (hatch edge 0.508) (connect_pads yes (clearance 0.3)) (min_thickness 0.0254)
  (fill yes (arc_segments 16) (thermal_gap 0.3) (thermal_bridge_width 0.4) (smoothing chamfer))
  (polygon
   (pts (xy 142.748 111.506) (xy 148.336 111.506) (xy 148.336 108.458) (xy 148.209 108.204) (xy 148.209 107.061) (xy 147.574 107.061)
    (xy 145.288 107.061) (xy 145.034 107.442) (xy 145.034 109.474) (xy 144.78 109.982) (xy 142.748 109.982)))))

